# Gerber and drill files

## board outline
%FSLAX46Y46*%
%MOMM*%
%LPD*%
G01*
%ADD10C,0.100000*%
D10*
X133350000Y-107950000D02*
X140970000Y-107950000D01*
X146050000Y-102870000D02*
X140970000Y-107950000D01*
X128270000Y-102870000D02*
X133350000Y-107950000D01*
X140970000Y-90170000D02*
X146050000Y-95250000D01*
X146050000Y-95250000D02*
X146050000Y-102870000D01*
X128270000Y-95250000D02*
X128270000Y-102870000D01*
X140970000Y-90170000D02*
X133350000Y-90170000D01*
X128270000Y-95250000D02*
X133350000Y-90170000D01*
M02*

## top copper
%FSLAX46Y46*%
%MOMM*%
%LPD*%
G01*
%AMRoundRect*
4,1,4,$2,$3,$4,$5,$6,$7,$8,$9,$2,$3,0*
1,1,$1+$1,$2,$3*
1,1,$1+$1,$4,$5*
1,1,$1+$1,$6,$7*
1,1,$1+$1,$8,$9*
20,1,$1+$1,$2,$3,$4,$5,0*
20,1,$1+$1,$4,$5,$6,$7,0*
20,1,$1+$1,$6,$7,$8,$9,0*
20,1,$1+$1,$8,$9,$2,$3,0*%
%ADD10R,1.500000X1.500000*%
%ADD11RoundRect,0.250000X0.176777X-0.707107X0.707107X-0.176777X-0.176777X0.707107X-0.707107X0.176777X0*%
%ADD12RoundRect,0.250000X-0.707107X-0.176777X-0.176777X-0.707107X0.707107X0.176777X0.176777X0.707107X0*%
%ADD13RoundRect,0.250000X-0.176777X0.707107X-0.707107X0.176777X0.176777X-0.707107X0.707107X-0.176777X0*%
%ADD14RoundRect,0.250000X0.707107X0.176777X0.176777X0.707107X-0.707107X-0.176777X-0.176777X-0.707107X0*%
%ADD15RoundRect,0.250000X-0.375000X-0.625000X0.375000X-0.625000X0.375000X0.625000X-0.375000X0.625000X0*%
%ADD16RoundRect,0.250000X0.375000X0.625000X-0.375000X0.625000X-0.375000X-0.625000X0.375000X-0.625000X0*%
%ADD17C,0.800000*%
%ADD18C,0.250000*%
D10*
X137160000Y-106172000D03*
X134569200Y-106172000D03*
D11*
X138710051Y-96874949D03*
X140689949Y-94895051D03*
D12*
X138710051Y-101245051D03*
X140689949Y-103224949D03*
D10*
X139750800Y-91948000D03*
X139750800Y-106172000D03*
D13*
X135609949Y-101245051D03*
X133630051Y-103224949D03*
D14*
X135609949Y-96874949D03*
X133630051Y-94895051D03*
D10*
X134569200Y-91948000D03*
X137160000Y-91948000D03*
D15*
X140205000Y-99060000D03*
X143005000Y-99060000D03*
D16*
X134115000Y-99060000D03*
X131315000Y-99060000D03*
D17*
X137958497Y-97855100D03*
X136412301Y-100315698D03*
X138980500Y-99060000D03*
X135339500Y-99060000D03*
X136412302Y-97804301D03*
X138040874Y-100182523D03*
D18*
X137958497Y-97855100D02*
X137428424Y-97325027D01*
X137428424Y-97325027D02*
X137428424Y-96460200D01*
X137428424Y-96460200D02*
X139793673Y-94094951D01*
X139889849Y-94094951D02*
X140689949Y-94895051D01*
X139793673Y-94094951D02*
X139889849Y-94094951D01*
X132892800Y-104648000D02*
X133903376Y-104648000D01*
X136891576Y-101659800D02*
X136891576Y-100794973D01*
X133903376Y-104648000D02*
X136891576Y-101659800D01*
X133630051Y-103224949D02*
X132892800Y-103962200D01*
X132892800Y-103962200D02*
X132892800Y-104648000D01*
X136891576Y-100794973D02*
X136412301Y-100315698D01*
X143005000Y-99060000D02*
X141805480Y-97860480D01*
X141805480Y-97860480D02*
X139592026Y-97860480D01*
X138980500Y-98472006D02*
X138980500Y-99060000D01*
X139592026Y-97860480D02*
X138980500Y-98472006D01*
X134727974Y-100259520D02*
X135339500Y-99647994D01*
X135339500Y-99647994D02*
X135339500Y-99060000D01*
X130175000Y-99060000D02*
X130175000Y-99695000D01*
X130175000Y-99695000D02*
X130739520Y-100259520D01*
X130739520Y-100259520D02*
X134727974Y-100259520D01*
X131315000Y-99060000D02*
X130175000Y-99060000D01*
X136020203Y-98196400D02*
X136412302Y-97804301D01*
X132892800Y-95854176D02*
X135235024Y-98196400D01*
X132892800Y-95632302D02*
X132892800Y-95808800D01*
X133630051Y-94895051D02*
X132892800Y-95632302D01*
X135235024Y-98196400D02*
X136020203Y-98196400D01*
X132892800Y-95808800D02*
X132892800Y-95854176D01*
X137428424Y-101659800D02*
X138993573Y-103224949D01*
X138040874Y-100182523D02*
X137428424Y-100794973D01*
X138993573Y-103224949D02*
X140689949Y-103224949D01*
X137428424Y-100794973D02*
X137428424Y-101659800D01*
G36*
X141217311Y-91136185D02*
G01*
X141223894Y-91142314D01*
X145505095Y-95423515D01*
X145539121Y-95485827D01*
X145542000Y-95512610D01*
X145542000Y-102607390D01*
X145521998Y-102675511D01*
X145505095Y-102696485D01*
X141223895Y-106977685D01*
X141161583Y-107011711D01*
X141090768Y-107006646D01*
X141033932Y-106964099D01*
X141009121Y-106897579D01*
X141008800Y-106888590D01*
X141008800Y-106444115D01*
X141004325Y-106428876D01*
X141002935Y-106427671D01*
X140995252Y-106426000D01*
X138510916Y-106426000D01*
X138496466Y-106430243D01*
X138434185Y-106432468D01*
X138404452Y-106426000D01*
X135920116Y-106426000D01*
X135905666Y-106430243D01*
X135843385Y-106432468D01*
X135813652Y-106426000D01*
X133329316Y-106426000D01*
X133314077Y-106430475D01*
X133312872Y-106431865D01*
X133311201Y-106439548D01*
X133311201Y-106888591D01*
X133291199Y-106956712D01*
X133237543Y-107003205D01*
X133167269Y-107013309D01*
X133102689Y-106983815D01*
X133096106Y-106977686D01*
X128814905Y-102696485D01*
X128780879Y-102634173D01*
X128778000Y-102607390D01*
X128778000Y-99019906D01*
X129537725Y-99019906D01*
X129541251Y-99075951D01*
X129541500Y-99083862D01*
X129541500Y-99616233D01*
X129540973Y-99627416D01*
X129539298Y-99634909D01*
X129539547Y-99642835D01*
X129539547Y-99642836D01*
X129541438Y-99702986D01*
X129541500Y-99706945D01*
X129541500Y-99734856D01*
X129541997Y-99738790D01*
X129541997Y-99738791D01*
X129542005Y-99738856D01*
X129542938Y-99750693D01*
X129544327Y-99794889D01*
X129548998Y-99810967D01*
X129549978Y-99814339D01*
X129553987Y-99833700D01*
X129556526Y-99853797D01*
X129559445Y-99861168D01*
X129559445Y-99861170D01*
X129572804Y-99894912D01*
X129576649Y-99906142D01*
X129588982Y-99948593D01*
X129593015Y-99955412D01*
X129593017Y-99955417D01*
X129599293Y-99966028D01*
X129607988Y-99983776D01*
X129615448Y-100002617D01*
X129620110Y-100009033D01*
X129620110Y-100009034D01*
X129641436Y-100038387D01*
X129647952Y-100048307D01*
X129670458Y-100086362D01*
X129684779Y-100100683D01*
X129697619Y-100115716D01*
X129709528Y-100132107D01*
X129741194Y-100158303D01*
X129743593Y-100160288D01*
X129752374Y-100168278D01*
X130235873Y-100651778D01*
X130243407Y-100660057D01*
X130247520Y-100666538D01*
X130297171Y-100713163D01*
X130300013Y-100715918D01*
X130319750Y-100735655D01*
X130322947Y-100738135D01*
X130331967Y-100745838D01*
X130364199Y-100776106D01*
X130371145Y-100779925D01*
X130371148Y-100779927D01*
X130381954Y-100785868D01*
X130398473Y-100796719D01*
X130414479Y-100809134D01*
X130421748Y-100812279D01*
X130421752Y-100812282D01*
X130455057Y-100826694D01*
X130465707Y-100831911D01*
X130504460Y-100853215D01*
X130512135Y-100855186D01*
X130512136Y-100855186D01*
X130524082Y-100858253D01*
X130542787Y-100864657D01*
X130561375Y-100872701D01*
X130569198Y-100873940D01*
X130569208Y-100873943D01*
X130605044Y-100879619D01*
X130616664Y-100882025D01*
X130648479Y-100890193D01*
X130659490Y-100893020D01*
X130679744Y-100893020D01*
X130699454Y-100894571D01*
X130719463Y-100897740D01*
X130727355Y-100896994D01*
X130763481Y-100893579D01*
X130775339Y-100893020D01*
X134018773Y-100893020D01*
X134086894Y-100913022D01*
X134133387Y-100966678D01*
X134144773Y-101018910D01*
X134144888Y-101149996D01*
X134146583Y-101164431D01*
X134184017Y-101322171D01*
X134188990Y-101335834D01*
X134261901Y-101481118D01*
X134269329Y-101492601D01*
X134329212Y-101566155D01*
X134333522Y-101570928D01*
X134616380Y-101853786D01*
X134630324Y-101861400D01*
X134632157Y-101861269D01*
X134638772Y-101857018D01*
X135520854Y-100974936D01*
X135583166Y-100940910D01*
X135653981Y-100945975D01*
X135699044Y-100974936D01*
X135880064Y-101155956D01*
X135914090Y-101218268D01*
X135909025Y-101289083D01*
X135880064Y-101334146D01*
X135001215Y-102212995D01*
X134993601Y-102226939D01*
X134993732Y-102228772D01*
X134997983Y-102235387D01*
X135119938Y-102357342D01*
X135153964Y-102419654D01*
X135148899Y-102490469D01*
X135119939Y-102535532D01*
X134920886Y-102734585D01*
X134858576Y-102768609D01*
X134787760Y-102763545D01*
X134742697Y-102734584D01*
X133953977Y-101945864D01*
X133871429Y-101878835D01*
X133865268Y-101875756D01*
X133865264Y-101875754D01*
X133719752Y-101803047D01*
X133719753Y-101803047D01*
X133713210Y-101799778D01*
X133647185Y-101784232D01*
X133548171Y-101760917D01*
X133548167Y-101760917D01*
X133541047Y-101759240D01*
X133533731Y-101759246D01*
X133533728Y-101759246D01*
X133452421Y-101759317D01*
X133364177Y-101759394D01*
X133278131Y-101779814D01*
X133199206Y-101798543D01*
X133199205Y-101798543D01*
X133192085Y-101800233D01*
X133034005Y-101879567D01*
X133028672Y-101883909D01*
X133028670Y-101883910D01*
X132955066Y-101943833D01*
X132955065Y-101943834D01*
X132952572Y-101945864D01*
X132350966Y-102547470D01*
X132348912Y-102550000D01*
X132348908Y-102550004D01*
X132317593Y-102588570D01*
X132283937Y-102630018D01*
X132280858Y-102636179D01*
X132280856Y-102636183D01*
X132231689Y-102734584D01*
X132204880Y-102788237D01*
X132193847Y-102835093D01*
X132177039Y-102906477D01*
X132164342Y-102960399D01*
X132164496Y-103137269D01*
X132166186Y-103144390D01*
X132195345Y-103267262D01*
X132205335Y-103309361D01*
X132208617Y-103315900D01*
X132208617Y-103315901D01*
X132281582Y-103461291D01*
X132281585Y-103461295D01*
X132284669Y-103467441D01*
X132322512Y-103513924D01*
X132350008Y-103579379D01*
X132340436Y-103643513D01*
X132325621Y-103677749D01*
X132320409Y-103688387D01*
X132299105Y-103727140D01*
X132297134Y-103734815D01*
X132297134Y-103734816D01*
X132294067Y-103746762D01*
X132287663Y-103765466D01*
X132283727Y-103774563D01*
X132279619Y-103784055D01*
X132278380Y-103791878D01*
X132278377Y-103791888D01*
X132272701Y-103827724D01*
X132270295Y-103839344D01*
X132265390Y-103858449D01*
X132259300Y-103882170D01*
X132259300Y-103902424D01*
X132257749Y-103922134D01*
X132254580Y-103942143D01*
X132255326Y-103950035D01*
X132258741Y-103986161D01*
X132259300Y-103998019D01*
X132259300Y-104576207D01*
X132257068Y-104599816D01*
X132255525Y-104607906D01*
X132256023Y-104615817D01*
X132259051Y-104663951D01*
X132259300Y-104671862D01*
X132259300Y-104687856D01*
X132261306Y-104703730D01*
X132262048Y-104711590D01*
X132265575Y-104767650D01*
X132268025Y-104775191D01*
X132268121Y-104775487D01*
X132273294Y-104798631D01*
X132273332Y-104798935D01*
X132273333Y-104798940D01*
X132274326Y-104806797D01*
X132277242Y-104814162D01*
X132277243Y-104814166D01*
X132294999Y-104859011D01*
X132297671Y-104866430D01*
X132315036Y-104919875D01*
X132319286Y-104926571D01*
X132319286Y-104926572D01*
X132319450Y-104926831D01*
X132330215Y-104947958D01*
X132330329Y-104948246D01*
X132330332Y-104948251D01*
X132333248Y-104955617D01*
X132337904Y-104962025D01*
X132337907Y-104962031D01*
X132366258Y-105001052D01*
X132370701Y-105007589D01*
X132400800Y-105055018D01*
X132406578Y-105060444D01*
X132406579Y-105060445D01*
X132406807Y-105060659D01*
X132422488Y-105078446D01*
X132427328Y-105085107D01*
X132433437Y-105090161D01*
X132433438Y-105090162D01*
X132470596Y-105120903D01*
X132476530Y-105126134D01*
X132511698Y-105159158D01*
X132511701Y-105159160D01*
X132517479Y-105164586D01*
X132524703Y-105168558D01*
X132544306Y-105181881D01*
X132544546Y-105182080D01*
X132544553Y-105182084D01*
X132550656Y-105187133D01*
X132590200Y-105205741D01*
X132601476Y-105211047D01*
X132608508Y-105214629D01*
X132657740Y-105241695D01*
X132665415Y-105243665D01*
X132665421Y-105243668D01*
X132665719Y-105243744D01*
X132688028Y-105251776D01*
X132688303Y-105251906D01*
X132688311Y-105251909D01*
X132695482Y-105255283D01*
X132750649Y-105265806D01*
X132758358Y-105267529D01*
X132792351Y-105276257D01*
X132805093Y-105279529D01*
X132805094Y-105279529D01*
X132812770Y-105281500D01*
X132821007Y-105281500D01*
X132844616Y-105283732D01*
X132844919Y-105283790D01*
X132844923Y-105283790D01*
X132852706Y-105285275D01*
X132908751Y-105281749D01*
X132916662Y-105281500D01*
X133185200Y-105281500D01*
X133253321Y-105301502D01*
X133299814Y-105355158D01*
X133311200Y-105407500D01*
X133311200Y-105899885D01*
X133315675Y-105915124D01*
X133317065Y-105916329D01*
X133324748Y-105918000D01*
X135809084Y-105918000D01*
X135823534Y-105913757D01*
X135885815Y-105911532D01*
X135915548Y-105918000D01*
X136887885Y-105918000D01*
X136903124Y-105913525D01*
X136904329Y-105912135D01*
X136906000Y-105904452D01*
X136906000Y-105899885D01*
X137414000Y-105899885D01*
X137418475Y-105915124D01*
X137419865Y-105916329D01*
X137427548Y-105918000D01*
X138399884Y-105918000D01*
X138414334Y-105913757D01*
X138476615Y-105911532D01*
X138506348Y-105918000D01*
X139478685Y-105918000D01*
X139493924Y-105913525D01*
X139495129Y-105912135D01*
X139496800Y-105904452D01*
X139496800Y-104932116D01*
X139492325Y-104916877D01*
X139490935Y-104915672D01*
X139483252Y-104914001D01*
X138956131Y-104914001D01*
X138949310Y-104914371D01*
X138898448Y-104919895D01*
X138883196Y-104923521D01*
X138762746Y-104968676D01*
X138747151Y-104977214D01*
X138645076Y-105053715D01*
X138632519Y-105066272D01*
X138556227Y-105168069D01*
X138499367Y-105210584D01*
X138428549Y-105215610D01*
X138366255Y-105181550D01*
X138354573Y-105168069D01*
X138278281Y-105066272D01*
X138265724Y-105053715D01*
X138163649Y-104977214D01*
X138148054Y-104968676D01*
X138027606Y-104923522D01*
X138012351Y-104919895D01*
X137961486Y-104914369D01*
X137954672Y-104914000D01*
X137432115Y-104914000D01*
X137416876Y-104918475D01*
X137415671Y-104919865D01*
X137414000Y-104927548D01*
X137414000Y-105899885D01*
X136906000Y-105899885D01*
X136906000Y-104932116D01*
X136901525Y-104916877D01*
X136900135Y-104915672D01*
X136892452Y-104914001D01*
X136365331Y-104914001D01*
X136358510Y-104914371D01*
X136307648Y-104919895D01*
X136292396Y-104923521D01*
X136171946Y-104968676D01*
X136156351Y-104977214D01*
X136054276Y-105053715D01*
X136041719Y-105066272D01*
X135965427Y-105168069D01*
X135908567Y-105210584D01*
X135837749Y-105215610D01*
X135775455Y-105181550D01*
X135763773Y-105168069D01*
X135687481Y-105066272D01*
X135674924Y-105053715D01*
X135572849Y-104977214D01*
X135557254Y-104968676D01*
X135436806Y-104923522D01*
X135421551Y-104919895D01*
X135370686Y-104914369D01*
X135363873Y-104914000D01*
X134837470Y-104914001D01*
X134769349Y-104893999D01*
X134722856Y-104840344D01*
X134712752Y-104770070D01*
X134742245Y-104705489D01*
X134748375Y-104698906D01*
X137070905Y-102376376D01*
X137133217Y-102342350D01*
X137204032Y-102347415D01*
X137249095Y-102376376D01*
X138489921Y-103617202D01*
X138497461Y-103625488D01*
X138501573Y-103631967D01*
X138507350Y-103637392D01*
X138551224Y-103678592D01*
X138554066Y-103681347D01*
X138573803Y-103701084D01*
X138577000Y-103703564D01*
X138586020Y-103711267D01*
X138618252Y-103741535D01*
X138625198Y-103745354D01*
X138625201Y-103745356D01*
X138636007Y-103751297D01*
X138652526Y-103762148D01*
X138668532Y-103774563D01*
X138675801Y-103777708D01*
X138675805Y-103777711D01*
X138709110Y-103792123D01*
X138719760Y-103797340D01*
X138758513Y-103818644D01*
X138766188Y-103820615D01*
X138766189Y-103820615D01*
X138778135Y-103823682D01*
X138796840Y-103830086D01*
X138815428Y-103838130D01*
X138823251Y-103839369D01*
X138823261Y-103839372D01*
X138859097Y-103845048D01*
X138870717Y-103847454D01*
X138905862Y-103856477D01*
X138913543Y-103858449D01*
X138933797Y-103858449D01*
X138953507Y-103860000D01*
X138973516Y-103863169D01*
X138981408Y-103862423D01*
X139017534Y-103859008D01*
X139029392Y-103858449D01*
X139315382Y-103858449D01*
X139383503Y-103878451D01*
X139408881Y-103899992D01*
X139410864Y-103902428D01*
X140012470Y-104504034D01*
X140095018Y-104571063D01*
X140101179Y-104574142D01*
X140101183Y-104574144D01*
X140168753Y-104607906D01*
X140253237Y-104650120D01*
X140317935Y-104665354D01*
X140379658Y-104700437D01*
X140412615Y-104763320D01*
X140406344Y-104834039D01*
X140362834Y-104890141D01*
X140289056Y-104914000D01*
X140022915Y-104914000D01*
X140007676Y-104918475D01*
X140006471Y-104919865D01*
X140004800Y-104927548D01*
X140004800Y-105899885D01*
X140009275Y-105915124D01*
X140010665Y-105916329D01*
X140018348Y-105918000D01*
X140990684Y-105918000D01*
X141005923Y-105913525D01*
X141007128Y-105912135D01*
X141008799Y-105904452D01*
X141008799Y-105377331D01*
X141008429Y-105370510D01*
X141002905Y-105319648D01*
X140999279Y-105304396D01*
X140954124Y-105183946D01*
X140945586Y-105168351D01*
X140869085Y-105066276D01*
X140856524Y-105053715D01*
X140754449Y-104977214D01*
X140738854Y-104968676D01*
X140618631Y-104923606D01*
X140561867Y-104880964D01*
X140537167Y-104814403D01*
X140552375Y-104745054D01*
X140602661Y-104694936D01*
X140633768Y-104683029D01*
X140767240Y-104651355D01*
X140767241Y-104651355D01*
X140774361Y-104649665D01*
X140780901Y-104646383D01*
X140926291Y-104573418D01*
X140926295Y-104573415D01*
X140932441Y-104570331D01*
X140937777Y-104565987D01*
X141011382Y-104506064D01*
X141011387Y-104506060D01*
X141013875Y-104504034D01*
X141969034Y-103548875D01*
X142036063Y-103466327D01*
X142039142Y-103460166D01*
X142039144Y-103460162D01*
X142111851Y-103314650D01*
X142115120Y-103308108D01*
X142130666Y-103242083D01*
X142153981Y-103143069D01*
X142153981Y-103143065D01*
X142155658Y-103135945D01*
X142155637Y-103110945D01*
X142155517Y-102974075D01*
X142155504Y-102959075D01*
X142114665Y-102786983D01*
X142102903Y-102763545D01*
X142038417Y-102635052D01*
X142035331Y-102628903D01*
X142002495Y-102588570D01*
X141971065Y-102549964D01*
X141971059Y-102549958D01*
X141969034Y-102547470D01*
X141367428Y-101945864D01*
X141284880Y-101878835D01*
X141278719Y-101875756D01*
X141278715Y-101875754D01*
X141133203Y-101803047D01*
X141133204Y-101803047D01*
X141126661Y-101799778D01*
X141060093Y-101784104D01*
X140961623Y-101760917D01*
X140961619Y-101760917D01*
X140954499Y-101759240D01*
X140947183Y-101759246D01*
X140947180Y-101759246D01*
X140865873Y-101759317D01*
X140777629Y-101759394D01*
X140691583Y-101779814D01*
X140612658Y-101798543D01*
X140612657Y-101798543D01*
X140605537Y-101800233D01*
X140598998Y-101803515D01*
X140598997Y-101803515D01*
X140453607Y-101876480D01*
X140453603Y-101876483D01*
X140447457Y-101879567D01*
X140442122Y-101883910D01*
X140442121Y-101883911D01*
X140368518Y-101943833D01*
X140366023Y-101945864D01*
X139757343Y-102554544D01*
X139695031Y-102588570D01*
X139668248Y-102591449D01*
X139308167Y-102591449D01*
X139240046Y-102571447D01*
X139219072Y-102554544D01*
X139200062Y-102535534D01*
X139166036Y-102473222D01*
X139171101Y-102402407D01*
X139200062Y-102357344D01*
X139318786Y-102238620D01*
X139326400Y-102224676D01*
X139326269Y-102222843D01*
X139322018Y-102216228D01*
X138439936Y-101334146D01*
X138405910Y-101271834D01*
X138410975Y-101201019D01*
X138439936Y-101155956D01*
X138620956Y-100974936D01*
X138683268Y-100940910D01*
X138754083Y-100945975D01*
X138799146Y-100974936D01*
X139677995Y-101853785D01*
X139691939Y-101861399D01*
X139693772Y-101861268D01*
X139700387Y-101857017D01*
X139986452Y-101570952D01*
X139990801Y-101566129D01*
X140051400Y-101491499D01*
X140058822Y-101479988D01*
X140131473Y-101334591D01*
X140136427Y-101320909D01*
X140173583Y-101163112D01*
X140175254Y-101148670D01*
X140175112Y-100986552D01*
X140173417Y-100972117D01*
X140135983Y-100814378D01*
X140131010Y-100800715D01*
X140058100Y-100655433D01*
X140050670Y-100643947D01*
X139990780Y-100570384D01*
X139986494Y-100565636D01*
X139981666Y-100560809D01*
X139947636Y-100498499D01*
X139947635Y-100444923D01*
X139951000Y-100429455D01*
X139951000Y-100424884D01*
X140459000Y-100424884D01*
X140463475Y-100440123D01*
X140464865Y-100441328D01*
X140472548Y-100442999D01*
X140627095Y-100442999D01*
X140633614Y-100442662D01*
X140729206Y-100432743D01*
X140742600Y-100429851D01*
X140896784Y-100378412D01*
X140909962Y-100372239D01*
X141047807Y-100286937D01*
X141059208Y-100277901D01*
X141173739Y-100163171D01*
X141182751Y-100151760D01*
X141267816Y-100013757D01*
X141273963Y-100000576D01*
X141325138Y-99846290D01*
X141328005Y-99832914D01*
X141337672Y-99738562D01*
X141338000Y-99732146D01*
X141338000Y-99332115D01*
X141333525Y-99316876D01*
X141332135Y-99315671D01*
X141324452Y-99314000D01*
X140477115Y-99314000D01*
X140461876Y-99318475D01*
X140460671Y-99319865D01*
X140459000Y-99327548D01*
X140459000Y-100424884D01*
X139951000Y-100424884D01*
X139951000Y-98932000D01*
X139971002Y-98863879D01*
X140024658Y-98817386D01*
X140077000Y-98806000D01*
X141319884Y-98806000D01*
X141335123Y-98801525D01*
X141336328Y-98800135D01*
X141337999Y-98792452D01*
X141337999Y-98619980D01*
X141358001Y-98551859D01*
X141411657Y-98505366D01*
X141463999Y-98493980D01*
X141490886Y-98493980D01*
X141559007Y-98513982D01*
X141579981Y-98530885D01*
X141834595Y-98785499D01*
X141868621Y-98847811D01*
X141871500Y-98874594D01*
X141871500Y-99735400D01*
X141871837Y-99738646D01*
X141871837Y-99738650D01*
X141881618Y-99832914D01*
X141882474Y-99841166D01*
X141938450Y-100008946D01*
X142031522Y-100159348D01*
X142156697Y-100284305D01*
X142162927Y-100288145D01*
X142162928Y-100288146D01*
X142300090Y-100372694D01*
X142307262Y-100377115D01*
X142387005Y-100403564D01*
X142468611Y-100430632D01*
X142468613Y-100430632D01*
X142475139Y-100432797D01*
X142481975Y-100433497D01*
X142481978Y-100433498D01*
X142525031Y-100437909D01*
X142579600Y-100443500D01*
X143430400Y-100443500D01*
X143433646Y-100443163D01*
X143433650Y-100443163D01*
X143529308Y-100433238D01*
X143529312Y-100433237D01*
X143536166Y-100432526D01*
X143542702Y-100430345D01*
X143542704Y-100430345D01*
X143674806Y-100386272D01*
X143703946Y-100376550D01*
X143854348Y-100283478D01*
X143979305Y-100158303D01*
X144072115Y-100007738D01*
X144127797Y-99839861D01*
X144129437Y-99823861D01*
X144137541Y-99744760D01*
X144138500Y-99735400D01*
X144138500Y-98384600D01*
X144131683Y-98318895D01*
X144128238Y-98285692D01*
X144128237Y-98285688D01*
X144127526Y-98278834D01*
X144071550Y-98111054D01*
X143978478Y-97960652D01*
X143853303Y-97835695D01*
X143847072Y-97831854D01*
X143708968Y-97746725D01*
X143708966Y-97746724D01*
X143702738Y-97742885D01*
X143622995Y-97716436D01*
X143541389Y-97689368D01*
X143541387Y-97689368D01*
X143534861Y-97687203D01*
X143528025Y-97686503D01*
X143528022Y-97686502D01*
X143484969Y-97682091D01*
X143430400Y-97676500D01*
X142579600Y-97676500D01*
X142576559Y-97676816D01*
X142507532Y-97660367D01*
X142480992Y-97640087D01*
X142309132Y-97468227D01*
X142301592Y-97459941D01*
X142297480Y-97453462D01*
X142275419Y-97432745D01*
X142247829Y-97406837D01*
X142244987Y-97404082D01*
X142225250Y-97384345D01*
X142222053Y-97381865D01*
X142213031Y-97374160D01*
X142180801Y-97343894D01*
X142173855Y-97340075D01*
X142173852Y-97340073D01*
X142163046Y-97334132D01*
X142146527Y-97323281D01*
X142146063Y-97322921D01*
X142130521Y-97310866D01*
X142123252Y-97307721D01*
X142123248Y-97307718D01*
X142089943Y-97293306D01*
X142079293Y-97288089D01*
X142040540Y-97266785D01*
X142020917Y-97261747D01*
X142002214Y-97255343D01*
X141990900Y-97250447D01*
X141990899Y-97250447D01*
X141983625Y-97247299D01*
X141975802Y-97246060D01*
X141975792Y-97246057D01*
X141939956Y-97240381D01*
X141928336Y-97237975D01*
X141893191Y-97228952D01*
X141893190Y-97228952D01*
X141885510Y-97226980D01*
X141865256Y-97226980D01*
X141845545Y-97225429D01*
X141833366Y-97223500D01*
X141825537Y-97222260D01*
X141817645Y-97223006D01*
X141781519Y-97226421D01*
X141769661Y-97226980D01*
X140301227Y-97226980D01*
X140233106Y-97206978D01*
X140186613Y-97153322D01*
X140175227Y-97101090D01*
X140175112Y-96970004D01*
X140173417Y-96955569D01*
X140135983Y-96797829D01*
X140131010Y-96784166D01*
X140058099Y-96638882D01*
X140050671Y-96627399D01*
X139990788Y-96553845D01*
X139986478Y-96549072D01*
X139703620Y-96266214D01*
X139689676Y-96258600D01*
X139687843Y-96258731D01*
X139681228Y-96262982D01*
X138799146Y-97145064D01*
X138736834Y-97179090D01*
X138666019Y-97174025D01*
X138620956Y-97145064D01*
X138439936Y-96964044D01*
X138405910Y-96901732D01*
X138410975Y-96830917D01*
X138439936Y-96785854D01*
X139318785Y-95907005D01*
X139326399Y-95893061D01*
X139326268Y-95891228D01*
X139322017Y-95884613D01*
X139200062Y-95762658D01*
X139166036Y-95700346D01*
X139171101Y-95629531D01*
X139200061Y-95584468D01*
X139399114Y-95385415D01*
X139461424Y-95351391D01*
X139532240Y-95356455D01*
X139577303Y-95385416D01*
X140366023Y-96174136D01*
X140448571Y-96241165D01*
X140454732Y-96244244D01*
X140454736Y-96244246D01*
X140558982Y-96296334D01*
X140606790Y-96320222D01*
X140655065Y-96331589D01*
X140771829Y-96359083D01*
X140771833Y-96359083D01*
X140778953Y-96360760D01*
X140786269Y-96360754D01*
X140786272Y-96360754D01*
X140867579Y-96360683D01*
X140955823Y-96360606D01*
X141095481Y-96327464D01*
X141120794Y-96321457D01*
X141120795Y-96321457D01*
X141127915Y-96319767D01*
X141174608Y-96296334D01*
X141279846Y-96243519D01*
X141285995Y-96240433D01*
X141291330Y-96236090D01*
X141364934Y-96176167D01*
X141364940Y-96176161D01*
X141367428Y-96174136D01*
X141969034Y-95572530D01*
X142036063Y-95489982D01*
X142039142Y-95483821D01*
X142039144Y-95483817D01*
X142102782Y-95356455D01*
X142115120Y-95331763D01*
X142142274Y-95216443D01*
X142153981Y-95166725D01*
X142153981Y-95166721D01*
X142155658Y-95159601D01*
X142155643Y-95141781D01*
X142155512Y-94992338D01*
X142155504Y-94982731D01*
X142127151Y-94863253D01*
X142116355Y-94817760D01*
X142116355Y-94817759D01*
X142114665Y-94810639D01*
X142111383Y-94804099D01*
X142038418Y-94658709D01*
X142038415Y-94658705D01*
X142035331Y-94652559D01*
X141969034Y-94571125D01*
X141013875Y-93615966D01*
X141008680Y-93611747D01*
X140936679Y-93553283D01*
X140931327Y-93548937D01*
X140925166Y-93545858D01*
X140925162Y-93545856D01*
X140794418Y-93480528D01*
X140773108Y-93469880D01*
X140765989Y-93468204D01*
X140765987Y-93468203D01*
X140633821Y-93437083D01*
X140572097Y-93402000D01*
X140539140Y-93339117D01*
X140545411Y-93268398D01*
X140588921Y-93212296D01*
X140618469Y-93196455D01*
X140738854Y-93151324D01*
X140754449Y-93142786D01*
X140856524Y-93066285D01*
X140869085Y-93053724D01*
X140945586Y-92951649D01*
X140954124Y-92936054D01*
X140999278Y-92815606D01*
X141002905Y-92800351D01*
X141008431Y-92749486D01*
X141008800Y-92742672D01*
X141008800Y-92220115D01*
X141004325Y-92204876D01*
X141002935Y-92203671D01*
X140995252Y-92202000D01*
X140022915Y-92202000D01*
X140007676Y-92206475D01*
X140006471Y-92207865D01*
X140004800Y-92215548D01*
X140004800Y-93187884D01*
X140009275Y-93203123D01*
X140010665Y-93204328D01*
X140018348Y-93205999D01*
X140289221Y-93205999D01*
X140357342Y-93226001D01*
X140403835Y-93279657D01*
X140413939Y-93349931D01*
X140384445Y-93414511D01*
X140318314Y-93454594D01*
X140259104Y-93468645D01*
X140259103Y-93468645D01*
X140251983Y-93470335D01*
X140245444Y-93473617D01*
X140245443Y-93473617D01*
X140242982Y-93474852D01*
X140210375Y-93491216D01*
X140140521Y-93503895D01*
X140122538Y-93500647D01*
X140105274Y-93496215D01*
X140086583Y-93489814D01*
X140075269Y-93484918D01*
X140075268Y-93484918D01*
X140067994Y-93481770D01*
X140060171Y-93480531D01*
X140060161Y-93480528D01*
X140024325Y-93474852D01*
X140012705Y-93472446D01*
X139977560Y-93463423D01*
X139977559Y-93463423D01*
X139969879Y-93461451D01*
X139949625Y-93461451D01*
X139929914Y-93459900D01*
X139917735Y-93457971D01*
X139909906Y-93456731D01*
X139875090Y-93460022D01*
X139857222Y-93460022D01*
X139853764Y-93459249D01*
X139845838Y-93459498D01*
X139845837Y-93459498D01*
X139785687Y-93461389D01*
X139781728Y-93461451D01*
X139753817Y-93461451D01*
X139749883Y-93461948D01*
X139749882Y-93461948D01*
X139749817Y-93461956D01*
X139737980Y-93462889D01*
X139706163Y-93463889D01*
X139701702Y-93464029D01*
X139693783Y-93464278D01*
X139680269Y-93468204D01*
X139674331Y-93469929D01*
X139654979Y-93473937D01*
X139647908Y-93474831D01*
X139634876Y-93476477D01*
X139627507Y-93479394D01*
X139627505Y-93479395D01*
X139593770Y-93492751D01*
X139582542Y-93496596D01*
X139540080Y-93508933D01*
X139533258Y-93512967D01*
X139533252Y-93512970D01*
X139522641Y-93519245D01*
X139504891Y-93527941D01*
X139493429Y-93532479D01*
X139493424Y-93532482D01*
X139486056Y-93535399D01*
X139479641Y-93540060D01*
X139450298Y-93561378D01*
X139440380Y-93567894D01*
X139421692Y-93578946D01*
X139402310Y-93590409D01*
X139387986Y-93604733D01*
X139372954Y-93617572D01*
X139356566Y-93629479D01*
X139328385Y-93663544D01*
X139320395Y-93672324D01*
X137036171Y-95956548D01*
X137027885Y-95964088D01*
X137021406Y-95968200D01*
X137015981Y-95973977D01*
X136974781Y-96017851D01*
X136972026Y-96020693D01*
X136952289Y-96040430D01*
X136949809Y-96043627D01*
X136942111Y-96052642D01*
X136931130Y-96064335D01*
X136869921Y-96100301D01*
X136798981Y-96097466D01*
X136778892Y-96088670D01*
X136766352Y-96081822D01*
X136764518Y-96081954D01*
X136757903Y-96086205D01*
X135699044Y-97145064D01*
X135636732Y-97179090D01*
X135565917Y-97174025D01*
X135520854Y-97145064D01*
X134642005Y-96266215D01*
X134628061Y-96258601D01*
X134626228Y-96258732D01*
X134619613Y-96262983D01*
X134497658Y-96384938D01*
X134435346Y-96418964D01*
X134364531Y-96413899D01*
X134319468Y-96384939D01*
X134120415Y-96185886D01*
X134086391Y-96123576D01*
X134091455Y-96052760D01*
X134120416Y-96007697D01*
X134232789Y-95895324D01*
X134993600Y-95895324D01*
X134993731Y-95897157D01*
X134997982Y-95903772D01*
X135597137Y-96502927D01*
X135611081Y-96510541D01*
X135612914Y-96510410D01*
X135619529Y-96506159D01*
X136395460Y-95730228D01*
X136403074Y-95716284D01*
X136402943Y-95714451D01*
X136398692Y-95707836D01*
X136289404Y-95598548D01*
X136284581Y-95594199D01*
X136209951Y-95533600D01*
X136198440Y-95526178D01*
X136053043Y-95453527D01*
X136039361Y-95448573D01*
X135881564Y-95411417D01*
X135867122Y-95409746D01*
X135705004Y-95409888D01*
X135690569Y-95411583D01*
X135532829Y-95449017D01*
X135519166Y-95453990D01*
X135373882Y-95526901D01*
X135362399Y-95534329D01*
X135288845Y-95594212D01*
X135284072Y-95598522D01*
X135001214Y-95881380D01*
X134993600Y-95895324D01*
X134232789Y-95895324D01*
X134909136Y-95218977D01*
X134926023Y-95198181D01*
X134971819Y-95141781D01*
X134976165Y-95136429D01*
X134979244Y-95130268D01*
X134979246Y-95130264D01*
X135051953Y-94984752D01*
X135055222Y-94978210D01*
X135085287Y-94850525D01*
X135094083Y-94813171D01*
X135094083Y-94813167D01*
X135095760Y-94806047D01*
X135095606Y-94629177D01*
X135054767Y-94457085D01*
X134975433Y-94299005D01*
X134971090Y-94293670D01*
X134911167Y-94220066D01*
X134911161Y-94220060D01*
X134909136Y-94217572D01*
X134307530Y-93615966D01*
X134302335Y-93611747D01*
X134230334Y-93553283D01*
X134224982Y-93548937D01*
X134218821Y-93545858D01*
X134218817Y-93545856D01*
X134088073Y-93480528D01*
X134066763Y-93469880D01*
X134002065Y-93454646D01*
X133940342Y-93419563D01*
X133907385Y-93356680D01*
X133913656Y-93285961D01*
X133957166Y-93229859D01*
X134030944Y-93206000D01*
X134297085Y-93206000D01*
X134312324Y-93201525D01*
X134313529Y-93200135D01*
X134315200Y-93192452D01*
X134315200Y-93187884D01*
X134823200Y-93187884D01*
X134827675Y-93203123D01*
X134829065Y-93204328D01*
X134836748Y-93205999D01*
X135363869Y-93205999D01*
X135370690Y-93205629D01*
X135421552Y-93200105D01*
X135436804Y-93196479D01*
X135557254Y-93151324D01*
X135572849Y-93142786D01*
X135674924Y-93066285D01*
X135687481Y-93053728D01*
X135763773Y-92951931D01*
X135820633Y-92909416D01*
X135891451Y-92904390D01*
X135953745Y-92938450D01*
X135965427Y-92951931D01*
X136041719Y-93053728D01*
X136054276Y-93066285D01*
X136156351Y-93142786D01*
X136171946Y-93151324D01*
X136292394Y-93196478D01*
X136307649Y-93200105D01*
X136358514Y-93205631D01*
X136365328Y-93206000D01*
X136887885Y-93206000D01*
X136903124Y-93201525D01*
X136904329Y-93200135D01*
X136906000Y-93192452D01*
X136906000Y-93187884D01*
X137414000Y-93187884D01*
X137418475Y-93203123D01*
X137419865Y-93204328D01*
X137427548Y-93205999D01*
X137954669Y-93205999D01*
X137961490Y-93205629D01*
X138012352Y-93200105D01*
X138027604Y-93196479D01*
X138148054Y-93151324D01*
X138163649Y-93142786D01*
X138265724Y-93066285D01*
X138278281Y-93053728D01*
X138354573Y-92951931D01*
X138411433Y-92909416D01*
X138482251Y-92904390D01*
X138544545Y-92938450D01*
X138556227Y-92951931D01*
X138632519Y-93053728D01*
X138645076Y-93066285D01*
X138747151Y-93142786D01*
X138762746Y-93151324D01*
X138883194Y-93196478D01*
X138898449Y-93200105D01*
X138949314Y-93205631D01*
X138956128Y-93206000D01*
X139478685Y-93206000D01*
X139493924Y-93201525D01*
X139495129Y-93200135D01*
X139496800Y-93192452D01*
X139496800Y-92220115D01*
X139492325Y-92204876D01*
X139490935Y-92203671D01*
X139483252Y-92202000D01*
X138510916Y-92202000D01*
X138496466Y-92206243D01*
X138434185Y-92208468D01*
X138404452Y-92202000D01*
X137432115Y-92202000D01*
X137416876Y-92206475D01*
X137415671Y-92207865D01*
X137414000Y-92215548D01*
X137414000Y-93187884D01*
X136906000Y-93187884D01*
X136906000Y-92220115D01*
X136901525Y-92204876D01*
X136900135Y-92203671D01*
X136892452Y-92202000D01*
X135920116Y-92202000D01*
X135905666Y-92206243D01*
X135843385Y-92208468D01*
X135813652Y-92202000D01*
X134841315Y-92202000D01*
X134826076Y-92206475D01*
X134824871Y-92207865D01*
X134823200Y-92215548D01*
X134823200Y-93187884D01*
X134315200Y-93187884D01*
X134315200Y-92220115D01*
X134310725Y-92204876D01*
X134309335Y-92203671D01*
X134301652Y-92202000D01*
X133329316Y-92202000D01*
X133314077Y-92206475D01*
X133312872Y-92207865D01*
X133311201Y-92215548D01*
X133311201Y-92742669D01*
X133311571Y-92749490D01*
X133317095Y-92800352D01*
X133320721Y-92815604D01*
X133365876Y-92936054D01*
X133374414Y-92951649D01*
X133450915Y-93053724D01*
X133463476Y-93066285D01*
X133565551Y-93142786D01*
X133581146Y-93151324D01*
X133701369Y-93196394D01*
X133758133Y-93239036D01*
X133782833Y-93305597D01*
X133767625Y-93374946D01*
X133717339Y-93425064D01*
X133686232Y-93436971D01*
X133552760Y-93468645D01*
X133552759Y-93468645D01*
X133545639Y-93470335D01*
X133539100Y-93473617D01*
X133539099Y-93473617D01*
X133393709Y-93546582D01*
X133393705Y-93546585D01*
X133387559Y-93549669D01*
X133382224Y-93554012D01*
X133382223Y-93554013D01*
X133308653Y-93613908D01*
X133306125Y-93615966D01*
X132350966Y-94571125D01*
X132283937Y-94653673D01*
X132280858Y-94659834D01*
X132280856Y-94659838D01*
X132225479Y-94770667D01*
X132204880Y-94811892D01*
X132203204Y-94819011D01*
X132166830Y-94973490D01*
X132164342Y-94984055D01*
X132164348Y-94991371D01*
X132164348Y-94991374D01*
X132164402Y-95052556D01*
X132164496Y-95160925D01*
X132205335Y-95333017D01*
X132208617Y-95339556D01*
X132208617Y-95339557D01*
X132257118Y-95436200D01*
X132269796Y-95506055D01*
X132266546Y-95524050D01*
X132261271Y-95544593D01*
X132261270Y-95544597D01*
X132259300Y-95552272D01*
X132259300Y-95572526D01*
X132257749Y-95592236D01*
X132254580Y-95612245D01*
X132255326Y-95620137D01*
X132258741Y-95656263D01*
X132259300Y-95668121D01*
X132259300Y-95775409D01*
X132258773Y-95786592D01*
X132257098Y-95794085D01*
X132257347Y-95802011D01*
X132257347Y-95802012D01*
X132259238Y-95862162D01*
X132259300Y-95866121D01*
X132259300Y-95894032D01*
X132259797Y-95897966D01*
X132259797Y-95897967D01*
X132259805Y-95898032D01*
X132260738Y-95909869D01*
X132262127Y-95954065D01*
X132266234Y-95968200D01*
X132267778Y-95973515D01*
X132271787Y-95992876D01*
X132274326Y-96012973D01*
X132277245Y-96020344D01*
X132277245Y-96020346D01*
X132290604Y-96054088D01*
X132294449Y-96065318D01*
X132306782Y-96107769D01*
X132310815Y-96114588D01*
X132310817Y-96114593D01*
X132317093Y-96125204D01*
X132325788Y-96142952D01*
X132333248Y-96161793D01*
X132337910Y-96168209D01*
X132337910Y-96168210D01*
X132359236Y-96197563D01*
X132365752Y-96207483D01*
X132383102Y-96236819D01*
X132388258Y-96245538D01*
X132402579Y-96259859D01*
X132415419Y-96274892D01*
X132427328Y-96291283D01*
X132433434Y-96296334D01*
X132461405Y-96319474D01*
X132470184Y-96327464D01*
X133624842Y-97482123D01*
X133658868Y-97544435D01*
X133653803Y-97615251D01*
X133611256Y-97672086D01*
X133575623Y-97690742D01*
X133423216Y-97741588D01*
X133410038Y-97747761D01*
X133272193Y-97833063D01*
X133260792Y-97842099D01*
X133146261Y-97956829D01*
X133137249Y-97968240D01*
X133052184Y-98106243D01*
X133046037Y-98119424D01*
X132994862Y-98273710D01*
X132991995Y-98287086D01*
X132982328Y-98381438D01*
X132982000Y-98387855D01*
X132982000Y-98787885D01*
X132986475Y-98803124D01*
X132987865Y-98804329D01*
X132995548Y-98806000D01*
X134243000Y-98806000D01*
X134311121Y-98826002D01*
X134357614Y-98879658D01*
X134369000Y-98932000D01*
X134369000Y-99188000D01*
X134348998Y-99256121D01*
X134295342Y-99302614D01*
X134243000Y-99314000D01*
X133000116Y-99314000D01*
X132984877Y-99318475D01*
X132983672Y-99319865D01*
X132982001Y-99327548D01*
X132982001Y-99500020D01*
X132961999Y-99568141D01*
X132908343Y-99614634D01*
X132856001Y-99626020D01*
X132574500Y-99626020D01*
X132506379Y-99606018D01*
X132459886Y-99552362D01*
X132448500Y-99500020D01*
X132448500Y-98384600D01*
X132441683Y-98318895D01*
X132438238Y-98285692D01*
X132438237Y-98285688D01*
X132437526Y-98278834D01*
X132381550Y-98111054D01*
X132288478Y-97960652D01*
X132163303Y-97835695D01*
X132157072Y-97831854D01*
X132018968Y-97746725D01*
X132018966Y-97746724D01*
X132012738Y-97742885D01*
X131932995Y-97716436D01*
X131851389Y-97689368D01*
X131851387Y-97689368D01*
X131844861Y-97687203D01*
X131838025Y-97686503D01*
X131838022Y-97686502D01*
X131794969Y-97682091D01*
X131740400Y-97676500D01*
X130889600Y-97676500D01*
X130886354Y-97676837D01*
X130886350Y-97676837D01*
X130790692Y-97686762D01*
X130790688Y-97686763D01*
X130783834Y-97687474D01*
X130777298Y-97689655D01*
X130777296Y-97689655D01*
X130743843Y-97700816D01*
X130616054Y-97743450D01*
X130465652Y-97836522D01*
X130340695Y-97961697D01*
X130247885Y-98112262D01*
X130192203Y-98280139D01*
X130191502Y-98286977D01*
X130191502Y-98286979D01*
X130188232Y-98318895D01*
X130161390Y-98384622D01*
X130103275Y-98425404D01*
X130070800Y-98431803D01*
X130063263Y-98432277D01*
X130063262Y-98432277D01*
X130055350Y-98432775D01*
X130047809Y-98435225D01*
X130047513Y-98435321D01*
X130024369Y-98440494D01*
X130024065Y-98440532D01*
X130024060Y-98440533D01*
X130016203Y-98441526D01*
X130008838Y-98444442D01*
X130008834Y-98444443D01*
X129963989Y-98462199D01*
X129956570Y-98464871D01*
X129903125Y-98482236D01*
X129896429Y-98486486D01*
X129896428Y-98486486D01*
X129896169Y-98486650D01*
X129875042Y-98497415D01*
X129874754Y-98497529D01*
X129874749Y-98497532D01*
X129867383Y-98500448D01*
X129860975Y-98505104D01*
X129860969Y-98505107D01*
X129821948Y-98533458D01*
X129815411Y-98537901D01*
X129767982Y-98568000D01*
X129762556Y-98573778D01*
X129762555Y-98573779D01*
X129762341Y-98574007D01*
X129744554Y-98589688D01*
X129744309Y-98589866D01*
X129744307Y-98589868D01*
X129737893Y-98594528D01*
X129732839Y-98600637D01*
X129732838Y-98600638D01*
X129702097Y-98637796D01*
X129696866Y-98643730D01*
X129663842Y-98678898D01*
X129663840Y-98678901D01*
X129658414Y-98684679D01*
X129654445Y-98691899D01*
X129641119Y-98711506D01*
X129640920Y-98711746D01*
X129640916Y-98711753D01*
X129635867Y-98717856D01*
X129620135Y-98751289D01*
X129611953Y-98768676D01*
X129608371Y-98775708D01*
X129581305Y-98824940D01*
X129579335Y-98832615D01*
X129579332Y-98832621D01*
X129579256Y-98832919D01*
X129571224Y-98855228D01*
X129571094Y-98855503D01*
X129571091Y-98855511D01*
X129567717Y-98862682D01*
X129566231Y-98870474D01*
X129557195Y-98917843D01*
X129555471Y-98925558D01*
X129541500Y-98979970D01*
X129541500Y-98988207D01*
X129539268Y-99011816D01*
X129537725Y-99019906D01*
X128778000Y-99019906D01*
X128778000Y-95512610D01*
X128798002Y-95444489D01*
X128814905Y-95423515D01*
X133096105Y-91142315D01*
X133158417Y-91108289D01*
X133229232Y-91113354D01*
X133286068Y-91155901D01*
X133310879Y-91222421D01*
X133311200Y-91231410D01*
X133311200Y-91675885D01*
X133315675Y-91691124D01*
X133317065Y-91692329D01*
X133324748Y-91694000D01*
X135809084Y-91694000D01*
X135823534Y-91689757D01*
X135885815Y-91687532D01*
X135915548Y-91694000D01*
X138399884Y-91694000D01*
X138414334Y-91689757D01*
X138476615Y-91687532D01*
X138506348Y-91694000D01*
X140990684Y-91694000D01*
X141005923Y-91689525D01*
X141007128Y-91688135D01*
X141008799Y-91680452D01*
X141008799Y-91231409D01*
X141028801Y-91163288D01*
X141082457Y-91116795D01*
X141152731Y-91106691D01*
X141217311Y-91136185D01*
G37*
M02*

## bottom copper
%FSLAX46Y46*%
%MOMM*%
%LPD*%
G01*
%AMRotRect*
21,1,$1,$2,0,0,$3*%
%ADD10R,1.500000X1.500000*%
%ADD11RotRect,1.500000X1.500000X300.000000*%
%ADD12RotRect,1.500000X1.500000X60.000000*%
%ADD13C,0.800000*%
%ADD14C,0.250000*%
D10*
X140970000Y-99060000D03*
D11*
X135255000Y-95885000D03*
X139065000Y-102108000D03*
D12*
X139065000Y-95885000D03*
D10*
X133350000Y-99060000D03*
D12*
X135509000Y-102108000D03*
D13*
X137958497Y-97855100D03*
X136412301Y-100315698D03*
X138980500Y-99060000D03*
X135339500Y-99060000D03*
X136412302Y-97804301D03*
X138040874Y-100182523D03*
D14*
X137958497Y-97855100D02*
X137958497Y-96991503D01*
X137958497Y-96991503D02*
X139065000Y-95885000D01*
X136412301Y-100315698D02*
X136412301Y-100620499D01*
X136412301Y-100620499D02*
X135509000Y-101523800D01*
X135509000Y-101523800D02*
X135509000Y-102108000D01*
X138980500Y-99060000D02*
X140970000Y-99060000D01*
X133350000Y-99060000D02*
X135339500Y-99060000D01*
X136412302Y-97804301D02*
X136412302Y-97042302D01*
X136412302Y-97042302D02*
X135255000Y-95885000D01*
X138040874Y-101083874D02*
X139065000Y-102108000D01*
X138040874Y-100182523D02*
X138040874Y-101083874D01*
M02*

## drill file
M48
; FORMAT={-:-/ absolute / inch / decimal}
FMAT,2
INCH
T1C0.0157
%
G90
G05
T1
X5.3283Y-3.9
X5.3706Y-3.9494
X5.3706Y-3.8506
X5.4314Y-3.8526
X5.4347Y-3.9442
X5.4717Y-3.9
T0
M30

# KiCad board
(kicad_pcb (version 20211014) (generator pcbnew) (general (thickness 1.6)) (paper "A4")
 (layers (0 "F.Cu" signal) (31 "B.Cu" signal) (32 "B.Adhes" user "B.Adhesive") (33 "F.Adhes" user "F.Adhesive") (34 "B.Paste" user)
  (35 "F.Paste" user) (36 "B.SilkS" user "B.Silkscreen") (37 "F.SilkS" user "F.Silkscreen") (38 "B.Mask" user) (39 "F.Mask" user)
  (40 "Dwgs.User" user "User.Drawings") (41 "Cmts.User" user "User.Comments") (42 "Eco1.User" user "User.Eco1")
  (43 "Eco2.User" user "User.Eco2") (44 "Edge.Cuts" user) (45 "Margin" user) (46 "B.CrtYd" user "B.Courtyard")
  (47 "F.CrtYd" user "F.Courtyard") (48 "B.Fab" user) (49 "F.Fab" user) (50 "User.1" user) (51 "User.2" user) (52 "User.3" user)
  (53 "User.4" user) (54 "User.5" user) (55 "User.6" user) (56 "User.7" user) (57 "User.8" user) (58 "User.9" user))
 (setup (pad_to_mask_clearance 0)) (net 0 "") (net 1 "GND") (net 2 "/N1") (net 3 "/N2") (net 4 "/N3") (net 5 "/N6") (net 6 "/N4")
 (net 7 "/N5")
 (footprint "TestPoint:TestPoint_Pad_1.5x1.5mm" (layer "F.Cu") (at 137.16 106.172)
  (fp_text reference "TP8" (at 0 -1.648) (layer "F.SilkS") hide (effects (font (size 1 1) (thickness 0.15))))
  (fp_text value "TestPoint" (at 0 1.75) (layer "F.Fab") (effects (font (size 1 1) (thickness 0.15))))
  (pad "1" smd rect locked (at 0 0) (size 1.5 1.5) (layers "F.Cu" "F.Mask") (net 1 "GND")))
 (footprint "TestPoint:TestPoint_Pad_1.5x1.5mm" (layer "F.Cu") (at 134.5692 106.172)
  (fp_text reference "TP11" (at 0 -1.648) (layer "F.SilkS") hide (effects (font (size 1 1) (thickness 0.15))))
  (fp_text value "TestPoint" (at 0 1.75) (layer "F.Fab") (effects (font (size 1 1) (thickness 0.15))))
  (pad "1" smd rect locked (at 0 0) (size 1.5 1.5) (layers "F.Cu" "F.Mask") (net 1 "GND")))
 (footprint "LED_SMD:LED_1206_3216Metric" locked (layer "F.Cu") (at 139.7 95.885 45)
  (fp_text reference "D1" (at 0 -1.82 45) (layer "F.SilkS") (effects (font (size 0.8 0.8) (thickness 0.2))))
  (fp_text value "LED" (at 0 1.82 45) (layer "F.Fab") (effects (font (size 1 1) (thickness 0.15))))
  (pad "1" smd roundrect locked (at -1.4 0 45) (size 1.25 1.75) (layers "F.Cu" "F.Paste" "F.Mask") (roundrect_rratio 0.2) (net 1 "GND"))
  (pad "2" smd roundrect locked (at 1.4 0 45) (size 1.25 1.75) (layers "F.Cu" "F.Paste" "F.Mask") (roundrect_rratio 0.2) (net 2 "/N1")))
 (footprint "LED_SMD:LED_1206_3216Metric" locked (layer "F.Cu") (at 139.7 102.235 -45)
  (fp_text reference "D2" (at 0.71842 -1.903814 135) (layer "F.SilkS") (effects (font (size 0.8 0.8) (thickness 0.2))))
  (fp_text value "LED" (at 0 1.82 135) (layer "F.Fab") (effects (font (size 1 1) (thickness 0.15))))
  (pad "1" smd roundrect locked (at -1.4 0 315) (size 1.25 1.75) (layers "F.Cu" "F.Paste" "F.Mask") (roundrect_rratio 0.2) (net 1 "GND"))
  (pad "2" smd roundrect locked (at 1.4 0 315) (size 1.25 1.75) (layers "F.Cu" "F.Paste" "F.Mask") (roundrect_rratio 0.2) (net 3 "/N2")))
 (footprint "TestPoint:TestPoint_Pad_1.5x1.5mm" (layer "F.Cu") (at 139.7508 91.948)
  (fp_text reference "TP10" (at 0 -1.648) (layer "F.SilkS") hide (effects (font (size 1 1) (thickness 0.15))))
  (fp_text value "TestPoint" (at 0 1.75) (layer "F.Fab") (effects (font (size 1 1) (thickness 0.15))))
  (pad "1" smd rect locked (at 0 0) (size 1.5 1.5) (layers "F.Cu" "F.Mask") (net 1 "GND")))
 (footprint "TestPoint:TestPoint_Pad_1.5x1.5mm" (layer "F.Cu") (at 139.7508 106.172)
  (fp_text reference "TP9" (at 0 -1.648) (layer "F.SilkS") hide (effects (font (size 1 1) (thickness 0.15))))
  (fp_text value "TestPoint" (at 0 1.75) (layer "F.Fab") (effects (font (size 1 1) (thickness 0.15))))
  (pad "1" smd rect locked (at 0 0) (size 1.5 1.5) (layers "F.Cu" "F.Mask") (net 1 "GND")))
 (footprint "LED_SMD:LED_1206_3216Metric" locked (layer "F.Cu") (at 134.62 102.235 -135)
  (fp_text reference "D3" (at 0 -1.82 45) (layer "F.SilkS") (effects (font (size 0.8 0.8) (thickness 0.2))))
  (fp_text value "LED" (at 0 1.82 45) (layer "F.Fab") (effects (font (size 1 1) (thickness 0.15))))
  (pad "1" smd roundrect locked (at -1.4 0 225) (size 1.25 1.75) (layers "F.Cu" "F.Paste" "F.Mask") (roundrect_rratio 0.2) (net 1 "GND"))
  (pad "2" smd roundrect locked (at 1.4 0 225) (size 1.25 1.75) (layers "F.Cu" "F.Paste" "F.Mask") (roundrect_rratio 0.2) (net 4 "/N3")))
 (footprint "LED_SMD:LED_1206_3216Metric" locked (layer "F.Cu") (at 134.62 95.885 135)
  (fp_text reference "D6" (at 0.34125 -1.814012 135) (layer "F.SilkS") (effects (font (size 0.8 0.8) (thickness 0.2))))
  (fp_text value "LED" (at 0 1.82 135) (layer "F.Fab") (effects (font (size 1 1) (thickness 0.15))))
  (pad "1" smd roundrect locked (at -1.4 0 135) (size 1.25 1.75) (layers "F.Cu" "F.Paste" "F.Mask") (roundrect_rratio 0.2) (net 1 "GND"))
  (pad "2" smd roundrect locked (at 1.4 0 135) (size 1.25 1.75) (layers "F.Cu" "F.Paste" "F.Mask") (roundrect_rratio 0.2) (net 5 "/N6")))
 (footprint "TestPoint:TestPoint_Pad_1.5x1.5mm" (layer "F.Cu") (at 134.5692 91.948)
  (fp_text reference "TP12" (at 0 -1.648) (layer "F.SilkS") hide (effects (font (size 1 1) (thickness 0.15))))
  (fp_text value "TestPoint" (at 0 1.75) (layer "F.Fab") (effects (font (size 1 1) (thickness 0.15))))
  (pad "1" smd rect locked (at 0 0) (size 1.5 1.5) (layers "F.Cu" "F.Mask") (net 1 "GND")))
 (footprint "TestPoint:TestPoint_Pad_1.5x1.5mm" (layer "F.Cu") (at 137.16 91.948)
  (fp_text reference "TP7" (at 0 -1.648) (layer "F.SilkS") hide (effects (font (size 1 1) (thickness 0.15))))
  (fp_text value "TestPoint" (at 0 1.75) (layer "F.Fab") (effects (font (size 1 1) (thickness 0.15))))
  (pad "1" smd rect locked (at 0 0) (size 1.5 1.5) (layers "F.Cu" "F.Mask") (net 1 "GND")))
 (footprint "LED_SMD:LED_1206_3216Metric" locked (layer "F.Cu") (at 141.605 99.06)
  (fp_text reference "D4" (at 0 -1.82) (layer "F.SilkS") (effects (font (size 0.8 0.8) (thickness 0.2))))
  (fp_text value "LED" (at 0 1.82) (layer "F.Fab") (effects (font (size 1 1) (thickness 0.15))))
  (pad "1" smd roundrect locked (at -1.4 0) (size 1.25 1.75) (layers "F.Cu" "F.Paste" "F.Mask") (roundrect_rratio 0.2) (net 1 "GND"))
  (pad "2" smd roundrect locked (at 1.4 0) (size 1.25 1.75) (layers "F.Cu" "F.Paste" "F.Mask") (roundrect_rratio 0.2) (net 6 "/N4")))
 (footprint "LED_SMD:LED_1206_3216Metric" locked (layer "F.Cu") (at 132.715 99.06 180)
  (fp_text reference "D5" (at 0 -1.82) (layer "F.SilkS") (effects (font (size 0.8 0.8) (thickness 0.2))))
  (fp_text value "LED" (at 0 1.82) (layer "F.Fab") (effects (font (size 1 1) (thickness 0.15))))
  (pad "1" smd roundrect locked (at -1.4 0 180) (size 1.25 1.75) (layers "F.Cu" "F.Paste" "F.Mask") (roundrect_rratio 0.2) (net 1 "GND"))
  (pad "2" smd roundrect locked (at 1.4 0 180) (size 1.25 1.75) (layers "F.Cu" "F.Paste" "F.Mask") (roundrect_rratio 0.2) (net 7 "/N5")))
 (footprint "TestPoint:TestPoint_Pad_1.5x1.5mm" (layer "B.Cu") (at 140.97 99.06 180)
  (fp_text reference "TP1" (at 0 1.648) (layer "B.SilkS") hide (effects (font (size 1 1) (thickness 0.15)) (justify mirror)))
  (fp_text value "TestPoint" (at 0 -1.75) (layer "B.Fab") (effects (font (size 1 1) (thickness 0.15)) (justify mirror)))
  (pad "1" smd rect locked (at 0 0 180) (size 1.5 1.5) (layers "B.Cu" "B.Mask") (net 6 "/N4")))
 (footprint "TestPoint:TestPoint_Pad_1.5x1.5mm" (layer "B.Cu") (at 135.255 95.885 -60)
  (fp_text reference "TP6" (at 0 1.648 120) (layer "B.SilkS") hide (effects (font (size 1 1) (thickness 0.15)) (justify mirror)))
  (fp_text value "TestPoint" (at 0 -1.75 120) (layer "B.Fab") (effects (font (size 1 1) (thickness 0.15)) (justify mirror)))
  (pad "1" smd rect locked (at 0 0 300) (size 1.5 1.5) (layers "B.Cu" "B.Mask") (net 5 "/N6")))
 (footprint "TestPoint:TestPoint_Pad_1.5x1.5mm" (layer "B.Cu") (at 139.065 102.108 -60)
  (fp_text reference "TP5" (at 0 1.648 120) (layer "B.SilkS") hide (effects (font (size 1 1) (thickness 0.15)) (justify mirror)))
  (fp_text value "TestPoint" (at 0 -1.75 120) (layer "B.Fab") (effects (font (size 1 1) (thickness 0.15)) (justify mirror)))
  (pad "1" smd rect locked (at 0 0 300) (size 1.5 1.5) (layers "B.Cu" "B.Mask") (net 3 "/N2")))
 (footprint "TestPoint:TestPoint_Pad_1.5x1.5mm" (layer "B.Cu") (at 139.065 95.885 60)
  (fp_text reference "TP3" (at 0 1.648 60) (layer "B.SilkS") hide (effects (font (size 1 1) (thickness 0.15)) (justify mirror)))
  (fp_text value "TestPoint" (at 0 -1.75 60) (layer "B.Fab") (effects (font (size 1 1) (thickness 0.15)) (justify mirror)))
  (pad "1" smd rect locked (at 0 0 60) (size 1.5 1.5) (layers "B.Cu" "B.Mask") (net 2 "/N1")))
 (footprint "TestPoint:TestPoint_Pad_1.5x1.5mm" (layer "B.Cu") (at 133.35 99.06 180)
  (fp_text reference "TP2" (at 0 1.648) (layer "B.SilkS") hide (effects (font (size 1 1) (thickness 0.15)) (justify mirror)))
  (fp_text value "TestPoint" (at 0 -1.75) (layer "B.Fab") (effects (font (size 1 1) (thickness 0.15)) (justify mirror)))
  (pad "1" smd rect locked (at 0 0 180) (size 1.5 1.5) (layers "B.Cu" "B.Mask") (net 7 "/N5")))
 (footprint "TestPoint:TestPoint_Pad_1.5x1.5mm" (layer "B.Cu") (at 135.509 102.108 60)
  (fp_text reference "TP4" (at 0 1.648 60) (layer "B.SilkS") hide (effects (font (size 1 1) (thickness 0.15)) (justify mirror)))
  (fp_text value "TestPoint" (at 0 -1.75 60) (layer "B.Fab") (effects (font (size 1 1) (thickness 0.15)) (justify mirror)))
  (pad "1" smd rect locked (at 0 0 60) (size 1.5 1.5) (layers "B.Cu" "B.Mask") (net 4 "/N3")))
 (gr_line (start 133.35 107.95) (end 140.97 107.95) (layer "Edge.Cuts") (width 0.1))
 (gr_line (start 146.05 102.87) (end 140.97 107.95) (layer "Edge.Cuts") (width 0.1))
 (gr_line (start 128.27 102.87) (end 133.35 107.95) (layer "Edge.Cuts") (width 0.1))
 (gr_line (start 140.97 90.17) (end 146.05 95.25) (layer "Edge.Cuts") (width 0.1))
 (gr_line (start 146.05 95.25) (end 146.05 102.87) (layer "Edge.Cuts") (width 0.1))
 (gr_line (start 128.27 95.25) (end 128.27 102.87) (layer "Edge.Cuts") (width 0.1))
 (gr_line (start 140.97 90.17) (end 133.35 90.17) (layer "Edge.Cuts") (width 0.1))
 (gr_line (start 128.27 95.25) (end 133.35 90.17) (layer "Edge.Cuts") (width 0.1))
 (segment (start 137.958497 97.8551) (end 137.428424 97.325027) (width 0.25) (layer "F.Cu") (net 2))
 (segment (start 137.428424 97.325027) (end 137.428424 96.4602) (width 0.25) (layer "F.Cu") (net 2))
 (segment (start 137.428424 96.4602) (end 139.793673 94.094951) (width 0.25) (layer "F.Cu") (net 2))
 (segment (start 139.889849 94.094951) (end 140.689949 94.895051) (width 0.25) (layer "F.Cu") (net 2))
 (segment (start 139.793673 94.094951) (end 139.889849 94.094951) (width 0.25) (layer "F.Cu") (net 2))
 (via (at 137.958497 97.8551) (size 0.8) (drill 0.4) (layers "F.Cu" "B.Cu") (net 2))
 (segment (start 137.958497 97.8551) (end 137.958497 96.991503) (width 0.25) (layer "B.Cu") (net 2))
 (segment (start 137.958497 96.991503) (end 139.065 95.885) (width 0.25) (layer "B.Cu") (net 2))
 (segment (start 132.8928 104.648) (end 133.903376 104.648) (width 0.25) (layer "F.Cu") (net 4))
 (segment (start 136.891576 101.6598) (end 136.891576 100.794973) (width 0.25) (layer "F.Cu") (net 4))
 (segment (start 133.903376 104.648) (end 136.891576 101.6598) (width 0.25) (layer "F.Cu") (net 4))
 (segment (start 133.630051 103.224949) (end 132.8928 103.9622) (width 0.25) (layer "F.Cu") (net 4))
 (segment (start 132.8928 103.9622) (end 132.8928 104.648) (width 0.25) (layer "F.Cu") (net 4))
 (segment (start 136.891576 100.794973) (end 136.412301 100.315698) (width 0.25) (layer "F.Cu") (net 4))
 (via (at 136.412301 100.315698) (size 0.8) (drill 0.4) (layers "F.Cu" "B.Cu") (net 4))
 (segment (start 136.412301 100.315698) (end 136.412301 100.620499) (width 0.25) (layer "B.Cu") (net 4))
 (segment (start 136.412301 100.620499) (end 135.509 101.5238) (width 0.25) (layer "B.Cu") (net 4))
 (segment (start 135.509 101.5238) (end 135.509 102.108) (width 0.25) (layer "B.Cu") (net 4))
 (segment (start 143.005 99.06) (end 141.80548 97.86048) (width 0.25) (layer "F.Cu") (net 6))
 (segment (start 141.80548 97.86048) (end 139.592026 97.86048) (width 0.25) (layer "F.Cu") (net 6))
 (segment (start 138.9805 98.472006) (end 138.9805 99.06) (width 0.25) (layer "F.Cu") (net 6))
 (segment (start 139.592026 97.86048) (end 138.9805 98.472006) (width 0.25) (layer "F.Cu") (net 6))
 (via (at 138.9805 99.06) (size 0.8) (drill 0.4) (layers "F.Cu" "B.Cu") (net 6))
 (segment (start 138.9805 99.06) (end 140.97 99.06) (width 0.25) (layer "B.Cu") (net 6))
 (segment (start 134.727974 100.25952) (end 135.3395 99.647994) (width 0.25) (layer "F.Cu") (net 7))
 (segment (start 135.3395 99.647994) (end 135.3395 99.06) (width 0.25) (layer "F.Cu") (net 7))
 (segment (start 130.175 99.06) (end 130.175 99.695) (width 0.25) (layer "F.Cu") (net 7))
 (segment (start 130.175 99.695) (end 130.73952 100.25952) (width 0.25) (layer "F.Cu") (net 7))
 (segment (start 130.73952 100.25952) (end 134.727974 100.25952) (width 0.25) (layer "F.Cu") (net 7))
 (segment (start 131.315 99.06) (end 130.175 99.06) (width 0.25) (layer "F.Cu") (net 7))
 (via (at 135.3395 99.06) (size 0.8) (drill 0.4) (layers "F.Cu" "B.Cu") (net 7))
 (segment (start 133.35 99.06) (end 135.3395 99.06) (width 0.25) (layer "B.Cu") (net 7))
 (segment (start 136.020203 98.1964) (end 136.412302 97.804301) (width 0.25) (layer "F.Cu") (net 5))
 (segment (start 132.8928 95.854176) (end 135.235024 98.1964) (width 0.25) (layer "F.Cu") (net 5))
 (segment (start 132.8928 95.632302) (end 132.8928 95.8088) (width 0.25) (layer "F.Cu") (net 5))
 (segment (start 133.630051 94.895051) (end 132.8928 95.632302) (width 0.25) (layer "F.Cu") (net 5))
 (segment (start 135.235024 98.1964) (end 136.020203 98.1964) (width 0.25) (layer "F.Cu") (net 5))
 (segment (start 132.8928 95.8088) (end 132.8928 95.854176) (width 0.25) (layer "F.Cu") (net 5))
 (via (at 136.412302 97.804301) (size 0.8) (drill 0.4) (layers "F.Cu" "B.Cu") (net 5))
 (segment (start 136.412302 97.804301) (end 136.412302 97.042302) (width 0.25) (layer "B.Cu") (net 5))
 (segment (start 136.412302 97.042302) (end 135.255 95.885) (width 0.25) (layer "B.Cu") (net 5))
 (segment (start 137.428424 101.6598) (end 138.993573 103.224949) (width 0.25) (layer "F.Cu") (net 3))
 (segment (start 138.040874 100.182523) (end 137.428424 100.794973) (width 0.25) (layer "F.Cu") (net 3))
 (segment (start 138.993573 103.224949) (end 140.689949 103.224949) (width 0.25) (layer "F.Cu") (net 3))
 (segment (start 137.428424 100.794973) (end 137.428424 101.6598) (width 0.25) (layer "F.Cu") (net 3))
 (via (at 138.040874 100.182523) (size 0.8) (drill 0.4) (layers "F.Cu" "B.Cu") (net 3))
 (segment (start 138.040874 101.083874) (end 139.065 102.108) (width 0.25) (layer "B.Cu") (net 3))
 (segment (start 138.040874 100.182523) (end 138.040874 101.083874) (width 0.25) (layer "B.Cu") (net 3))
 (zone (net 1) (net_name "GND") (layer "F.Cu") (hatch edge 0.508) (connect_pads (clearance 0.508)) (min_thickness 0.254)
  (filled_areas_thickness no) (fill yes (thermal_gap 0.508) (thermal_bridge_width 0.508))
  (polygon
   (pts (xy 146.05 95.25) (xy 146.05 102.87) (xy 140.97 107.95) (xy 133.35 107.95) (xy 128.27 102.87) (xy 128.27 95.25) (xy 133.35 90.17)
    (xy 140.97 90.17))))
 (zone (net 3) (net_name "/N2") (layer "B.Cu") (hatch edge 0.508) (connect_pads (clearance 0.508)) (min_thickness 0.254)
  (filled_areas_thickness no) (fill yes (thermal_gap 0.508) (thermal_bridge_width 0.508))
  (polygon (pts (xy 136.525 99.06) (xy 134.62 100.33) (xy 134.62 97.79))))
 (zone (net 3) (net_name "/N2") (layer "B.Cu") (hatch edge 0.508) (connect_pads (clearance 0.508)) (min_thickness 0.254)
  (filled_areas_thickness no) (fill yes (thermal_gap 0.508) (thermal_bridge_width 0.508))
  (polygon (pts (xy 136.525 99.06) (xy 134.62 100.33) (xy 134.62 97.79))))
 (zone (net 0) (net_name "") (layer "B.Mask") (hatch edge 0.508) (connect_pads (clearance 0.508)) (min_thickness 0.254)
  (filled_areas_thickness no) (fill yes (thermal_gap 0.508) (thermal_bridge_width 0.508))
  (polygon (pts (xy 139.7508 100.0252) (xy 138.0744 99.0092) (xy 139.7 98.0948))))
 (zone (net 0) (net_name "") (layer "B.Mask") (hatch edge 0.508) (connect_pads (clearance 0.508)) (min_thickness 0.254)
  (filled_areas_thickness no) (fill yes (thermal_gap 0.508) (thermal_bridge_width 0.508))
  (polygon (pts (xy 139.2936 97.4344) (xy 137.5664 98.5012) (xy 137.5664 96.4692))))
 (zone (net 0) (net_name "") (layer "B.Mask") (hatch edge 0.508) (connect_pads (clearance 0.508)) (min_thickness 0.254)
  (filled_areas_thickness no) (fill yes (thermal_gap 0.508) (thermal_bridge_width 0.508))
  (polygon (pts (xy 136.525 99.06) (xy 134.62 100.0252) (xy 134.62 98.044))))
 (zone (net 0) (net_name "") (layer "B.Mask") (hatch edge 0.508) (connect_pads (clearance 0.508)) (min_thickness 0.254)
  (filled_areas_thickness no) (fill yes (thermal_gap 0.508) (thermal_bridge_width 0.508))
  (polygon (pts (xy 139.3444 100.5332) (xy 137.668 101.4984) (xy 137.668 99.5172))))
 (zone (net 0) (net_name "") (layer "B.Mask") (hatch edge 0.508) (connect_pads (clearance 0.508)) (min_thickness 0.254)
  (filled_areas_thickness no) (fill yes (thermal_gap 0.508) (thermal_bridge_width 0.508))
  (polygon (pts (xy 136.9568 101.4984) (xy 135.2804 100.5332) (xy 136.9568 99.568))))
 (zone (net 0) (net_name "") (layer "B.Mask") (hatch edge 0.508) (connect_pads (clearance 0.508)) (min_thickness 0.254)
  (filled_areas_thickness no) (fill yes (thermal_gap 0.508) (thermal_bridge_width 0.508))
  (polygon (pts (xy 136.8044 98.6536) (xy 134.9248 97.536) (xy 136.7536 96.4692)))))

